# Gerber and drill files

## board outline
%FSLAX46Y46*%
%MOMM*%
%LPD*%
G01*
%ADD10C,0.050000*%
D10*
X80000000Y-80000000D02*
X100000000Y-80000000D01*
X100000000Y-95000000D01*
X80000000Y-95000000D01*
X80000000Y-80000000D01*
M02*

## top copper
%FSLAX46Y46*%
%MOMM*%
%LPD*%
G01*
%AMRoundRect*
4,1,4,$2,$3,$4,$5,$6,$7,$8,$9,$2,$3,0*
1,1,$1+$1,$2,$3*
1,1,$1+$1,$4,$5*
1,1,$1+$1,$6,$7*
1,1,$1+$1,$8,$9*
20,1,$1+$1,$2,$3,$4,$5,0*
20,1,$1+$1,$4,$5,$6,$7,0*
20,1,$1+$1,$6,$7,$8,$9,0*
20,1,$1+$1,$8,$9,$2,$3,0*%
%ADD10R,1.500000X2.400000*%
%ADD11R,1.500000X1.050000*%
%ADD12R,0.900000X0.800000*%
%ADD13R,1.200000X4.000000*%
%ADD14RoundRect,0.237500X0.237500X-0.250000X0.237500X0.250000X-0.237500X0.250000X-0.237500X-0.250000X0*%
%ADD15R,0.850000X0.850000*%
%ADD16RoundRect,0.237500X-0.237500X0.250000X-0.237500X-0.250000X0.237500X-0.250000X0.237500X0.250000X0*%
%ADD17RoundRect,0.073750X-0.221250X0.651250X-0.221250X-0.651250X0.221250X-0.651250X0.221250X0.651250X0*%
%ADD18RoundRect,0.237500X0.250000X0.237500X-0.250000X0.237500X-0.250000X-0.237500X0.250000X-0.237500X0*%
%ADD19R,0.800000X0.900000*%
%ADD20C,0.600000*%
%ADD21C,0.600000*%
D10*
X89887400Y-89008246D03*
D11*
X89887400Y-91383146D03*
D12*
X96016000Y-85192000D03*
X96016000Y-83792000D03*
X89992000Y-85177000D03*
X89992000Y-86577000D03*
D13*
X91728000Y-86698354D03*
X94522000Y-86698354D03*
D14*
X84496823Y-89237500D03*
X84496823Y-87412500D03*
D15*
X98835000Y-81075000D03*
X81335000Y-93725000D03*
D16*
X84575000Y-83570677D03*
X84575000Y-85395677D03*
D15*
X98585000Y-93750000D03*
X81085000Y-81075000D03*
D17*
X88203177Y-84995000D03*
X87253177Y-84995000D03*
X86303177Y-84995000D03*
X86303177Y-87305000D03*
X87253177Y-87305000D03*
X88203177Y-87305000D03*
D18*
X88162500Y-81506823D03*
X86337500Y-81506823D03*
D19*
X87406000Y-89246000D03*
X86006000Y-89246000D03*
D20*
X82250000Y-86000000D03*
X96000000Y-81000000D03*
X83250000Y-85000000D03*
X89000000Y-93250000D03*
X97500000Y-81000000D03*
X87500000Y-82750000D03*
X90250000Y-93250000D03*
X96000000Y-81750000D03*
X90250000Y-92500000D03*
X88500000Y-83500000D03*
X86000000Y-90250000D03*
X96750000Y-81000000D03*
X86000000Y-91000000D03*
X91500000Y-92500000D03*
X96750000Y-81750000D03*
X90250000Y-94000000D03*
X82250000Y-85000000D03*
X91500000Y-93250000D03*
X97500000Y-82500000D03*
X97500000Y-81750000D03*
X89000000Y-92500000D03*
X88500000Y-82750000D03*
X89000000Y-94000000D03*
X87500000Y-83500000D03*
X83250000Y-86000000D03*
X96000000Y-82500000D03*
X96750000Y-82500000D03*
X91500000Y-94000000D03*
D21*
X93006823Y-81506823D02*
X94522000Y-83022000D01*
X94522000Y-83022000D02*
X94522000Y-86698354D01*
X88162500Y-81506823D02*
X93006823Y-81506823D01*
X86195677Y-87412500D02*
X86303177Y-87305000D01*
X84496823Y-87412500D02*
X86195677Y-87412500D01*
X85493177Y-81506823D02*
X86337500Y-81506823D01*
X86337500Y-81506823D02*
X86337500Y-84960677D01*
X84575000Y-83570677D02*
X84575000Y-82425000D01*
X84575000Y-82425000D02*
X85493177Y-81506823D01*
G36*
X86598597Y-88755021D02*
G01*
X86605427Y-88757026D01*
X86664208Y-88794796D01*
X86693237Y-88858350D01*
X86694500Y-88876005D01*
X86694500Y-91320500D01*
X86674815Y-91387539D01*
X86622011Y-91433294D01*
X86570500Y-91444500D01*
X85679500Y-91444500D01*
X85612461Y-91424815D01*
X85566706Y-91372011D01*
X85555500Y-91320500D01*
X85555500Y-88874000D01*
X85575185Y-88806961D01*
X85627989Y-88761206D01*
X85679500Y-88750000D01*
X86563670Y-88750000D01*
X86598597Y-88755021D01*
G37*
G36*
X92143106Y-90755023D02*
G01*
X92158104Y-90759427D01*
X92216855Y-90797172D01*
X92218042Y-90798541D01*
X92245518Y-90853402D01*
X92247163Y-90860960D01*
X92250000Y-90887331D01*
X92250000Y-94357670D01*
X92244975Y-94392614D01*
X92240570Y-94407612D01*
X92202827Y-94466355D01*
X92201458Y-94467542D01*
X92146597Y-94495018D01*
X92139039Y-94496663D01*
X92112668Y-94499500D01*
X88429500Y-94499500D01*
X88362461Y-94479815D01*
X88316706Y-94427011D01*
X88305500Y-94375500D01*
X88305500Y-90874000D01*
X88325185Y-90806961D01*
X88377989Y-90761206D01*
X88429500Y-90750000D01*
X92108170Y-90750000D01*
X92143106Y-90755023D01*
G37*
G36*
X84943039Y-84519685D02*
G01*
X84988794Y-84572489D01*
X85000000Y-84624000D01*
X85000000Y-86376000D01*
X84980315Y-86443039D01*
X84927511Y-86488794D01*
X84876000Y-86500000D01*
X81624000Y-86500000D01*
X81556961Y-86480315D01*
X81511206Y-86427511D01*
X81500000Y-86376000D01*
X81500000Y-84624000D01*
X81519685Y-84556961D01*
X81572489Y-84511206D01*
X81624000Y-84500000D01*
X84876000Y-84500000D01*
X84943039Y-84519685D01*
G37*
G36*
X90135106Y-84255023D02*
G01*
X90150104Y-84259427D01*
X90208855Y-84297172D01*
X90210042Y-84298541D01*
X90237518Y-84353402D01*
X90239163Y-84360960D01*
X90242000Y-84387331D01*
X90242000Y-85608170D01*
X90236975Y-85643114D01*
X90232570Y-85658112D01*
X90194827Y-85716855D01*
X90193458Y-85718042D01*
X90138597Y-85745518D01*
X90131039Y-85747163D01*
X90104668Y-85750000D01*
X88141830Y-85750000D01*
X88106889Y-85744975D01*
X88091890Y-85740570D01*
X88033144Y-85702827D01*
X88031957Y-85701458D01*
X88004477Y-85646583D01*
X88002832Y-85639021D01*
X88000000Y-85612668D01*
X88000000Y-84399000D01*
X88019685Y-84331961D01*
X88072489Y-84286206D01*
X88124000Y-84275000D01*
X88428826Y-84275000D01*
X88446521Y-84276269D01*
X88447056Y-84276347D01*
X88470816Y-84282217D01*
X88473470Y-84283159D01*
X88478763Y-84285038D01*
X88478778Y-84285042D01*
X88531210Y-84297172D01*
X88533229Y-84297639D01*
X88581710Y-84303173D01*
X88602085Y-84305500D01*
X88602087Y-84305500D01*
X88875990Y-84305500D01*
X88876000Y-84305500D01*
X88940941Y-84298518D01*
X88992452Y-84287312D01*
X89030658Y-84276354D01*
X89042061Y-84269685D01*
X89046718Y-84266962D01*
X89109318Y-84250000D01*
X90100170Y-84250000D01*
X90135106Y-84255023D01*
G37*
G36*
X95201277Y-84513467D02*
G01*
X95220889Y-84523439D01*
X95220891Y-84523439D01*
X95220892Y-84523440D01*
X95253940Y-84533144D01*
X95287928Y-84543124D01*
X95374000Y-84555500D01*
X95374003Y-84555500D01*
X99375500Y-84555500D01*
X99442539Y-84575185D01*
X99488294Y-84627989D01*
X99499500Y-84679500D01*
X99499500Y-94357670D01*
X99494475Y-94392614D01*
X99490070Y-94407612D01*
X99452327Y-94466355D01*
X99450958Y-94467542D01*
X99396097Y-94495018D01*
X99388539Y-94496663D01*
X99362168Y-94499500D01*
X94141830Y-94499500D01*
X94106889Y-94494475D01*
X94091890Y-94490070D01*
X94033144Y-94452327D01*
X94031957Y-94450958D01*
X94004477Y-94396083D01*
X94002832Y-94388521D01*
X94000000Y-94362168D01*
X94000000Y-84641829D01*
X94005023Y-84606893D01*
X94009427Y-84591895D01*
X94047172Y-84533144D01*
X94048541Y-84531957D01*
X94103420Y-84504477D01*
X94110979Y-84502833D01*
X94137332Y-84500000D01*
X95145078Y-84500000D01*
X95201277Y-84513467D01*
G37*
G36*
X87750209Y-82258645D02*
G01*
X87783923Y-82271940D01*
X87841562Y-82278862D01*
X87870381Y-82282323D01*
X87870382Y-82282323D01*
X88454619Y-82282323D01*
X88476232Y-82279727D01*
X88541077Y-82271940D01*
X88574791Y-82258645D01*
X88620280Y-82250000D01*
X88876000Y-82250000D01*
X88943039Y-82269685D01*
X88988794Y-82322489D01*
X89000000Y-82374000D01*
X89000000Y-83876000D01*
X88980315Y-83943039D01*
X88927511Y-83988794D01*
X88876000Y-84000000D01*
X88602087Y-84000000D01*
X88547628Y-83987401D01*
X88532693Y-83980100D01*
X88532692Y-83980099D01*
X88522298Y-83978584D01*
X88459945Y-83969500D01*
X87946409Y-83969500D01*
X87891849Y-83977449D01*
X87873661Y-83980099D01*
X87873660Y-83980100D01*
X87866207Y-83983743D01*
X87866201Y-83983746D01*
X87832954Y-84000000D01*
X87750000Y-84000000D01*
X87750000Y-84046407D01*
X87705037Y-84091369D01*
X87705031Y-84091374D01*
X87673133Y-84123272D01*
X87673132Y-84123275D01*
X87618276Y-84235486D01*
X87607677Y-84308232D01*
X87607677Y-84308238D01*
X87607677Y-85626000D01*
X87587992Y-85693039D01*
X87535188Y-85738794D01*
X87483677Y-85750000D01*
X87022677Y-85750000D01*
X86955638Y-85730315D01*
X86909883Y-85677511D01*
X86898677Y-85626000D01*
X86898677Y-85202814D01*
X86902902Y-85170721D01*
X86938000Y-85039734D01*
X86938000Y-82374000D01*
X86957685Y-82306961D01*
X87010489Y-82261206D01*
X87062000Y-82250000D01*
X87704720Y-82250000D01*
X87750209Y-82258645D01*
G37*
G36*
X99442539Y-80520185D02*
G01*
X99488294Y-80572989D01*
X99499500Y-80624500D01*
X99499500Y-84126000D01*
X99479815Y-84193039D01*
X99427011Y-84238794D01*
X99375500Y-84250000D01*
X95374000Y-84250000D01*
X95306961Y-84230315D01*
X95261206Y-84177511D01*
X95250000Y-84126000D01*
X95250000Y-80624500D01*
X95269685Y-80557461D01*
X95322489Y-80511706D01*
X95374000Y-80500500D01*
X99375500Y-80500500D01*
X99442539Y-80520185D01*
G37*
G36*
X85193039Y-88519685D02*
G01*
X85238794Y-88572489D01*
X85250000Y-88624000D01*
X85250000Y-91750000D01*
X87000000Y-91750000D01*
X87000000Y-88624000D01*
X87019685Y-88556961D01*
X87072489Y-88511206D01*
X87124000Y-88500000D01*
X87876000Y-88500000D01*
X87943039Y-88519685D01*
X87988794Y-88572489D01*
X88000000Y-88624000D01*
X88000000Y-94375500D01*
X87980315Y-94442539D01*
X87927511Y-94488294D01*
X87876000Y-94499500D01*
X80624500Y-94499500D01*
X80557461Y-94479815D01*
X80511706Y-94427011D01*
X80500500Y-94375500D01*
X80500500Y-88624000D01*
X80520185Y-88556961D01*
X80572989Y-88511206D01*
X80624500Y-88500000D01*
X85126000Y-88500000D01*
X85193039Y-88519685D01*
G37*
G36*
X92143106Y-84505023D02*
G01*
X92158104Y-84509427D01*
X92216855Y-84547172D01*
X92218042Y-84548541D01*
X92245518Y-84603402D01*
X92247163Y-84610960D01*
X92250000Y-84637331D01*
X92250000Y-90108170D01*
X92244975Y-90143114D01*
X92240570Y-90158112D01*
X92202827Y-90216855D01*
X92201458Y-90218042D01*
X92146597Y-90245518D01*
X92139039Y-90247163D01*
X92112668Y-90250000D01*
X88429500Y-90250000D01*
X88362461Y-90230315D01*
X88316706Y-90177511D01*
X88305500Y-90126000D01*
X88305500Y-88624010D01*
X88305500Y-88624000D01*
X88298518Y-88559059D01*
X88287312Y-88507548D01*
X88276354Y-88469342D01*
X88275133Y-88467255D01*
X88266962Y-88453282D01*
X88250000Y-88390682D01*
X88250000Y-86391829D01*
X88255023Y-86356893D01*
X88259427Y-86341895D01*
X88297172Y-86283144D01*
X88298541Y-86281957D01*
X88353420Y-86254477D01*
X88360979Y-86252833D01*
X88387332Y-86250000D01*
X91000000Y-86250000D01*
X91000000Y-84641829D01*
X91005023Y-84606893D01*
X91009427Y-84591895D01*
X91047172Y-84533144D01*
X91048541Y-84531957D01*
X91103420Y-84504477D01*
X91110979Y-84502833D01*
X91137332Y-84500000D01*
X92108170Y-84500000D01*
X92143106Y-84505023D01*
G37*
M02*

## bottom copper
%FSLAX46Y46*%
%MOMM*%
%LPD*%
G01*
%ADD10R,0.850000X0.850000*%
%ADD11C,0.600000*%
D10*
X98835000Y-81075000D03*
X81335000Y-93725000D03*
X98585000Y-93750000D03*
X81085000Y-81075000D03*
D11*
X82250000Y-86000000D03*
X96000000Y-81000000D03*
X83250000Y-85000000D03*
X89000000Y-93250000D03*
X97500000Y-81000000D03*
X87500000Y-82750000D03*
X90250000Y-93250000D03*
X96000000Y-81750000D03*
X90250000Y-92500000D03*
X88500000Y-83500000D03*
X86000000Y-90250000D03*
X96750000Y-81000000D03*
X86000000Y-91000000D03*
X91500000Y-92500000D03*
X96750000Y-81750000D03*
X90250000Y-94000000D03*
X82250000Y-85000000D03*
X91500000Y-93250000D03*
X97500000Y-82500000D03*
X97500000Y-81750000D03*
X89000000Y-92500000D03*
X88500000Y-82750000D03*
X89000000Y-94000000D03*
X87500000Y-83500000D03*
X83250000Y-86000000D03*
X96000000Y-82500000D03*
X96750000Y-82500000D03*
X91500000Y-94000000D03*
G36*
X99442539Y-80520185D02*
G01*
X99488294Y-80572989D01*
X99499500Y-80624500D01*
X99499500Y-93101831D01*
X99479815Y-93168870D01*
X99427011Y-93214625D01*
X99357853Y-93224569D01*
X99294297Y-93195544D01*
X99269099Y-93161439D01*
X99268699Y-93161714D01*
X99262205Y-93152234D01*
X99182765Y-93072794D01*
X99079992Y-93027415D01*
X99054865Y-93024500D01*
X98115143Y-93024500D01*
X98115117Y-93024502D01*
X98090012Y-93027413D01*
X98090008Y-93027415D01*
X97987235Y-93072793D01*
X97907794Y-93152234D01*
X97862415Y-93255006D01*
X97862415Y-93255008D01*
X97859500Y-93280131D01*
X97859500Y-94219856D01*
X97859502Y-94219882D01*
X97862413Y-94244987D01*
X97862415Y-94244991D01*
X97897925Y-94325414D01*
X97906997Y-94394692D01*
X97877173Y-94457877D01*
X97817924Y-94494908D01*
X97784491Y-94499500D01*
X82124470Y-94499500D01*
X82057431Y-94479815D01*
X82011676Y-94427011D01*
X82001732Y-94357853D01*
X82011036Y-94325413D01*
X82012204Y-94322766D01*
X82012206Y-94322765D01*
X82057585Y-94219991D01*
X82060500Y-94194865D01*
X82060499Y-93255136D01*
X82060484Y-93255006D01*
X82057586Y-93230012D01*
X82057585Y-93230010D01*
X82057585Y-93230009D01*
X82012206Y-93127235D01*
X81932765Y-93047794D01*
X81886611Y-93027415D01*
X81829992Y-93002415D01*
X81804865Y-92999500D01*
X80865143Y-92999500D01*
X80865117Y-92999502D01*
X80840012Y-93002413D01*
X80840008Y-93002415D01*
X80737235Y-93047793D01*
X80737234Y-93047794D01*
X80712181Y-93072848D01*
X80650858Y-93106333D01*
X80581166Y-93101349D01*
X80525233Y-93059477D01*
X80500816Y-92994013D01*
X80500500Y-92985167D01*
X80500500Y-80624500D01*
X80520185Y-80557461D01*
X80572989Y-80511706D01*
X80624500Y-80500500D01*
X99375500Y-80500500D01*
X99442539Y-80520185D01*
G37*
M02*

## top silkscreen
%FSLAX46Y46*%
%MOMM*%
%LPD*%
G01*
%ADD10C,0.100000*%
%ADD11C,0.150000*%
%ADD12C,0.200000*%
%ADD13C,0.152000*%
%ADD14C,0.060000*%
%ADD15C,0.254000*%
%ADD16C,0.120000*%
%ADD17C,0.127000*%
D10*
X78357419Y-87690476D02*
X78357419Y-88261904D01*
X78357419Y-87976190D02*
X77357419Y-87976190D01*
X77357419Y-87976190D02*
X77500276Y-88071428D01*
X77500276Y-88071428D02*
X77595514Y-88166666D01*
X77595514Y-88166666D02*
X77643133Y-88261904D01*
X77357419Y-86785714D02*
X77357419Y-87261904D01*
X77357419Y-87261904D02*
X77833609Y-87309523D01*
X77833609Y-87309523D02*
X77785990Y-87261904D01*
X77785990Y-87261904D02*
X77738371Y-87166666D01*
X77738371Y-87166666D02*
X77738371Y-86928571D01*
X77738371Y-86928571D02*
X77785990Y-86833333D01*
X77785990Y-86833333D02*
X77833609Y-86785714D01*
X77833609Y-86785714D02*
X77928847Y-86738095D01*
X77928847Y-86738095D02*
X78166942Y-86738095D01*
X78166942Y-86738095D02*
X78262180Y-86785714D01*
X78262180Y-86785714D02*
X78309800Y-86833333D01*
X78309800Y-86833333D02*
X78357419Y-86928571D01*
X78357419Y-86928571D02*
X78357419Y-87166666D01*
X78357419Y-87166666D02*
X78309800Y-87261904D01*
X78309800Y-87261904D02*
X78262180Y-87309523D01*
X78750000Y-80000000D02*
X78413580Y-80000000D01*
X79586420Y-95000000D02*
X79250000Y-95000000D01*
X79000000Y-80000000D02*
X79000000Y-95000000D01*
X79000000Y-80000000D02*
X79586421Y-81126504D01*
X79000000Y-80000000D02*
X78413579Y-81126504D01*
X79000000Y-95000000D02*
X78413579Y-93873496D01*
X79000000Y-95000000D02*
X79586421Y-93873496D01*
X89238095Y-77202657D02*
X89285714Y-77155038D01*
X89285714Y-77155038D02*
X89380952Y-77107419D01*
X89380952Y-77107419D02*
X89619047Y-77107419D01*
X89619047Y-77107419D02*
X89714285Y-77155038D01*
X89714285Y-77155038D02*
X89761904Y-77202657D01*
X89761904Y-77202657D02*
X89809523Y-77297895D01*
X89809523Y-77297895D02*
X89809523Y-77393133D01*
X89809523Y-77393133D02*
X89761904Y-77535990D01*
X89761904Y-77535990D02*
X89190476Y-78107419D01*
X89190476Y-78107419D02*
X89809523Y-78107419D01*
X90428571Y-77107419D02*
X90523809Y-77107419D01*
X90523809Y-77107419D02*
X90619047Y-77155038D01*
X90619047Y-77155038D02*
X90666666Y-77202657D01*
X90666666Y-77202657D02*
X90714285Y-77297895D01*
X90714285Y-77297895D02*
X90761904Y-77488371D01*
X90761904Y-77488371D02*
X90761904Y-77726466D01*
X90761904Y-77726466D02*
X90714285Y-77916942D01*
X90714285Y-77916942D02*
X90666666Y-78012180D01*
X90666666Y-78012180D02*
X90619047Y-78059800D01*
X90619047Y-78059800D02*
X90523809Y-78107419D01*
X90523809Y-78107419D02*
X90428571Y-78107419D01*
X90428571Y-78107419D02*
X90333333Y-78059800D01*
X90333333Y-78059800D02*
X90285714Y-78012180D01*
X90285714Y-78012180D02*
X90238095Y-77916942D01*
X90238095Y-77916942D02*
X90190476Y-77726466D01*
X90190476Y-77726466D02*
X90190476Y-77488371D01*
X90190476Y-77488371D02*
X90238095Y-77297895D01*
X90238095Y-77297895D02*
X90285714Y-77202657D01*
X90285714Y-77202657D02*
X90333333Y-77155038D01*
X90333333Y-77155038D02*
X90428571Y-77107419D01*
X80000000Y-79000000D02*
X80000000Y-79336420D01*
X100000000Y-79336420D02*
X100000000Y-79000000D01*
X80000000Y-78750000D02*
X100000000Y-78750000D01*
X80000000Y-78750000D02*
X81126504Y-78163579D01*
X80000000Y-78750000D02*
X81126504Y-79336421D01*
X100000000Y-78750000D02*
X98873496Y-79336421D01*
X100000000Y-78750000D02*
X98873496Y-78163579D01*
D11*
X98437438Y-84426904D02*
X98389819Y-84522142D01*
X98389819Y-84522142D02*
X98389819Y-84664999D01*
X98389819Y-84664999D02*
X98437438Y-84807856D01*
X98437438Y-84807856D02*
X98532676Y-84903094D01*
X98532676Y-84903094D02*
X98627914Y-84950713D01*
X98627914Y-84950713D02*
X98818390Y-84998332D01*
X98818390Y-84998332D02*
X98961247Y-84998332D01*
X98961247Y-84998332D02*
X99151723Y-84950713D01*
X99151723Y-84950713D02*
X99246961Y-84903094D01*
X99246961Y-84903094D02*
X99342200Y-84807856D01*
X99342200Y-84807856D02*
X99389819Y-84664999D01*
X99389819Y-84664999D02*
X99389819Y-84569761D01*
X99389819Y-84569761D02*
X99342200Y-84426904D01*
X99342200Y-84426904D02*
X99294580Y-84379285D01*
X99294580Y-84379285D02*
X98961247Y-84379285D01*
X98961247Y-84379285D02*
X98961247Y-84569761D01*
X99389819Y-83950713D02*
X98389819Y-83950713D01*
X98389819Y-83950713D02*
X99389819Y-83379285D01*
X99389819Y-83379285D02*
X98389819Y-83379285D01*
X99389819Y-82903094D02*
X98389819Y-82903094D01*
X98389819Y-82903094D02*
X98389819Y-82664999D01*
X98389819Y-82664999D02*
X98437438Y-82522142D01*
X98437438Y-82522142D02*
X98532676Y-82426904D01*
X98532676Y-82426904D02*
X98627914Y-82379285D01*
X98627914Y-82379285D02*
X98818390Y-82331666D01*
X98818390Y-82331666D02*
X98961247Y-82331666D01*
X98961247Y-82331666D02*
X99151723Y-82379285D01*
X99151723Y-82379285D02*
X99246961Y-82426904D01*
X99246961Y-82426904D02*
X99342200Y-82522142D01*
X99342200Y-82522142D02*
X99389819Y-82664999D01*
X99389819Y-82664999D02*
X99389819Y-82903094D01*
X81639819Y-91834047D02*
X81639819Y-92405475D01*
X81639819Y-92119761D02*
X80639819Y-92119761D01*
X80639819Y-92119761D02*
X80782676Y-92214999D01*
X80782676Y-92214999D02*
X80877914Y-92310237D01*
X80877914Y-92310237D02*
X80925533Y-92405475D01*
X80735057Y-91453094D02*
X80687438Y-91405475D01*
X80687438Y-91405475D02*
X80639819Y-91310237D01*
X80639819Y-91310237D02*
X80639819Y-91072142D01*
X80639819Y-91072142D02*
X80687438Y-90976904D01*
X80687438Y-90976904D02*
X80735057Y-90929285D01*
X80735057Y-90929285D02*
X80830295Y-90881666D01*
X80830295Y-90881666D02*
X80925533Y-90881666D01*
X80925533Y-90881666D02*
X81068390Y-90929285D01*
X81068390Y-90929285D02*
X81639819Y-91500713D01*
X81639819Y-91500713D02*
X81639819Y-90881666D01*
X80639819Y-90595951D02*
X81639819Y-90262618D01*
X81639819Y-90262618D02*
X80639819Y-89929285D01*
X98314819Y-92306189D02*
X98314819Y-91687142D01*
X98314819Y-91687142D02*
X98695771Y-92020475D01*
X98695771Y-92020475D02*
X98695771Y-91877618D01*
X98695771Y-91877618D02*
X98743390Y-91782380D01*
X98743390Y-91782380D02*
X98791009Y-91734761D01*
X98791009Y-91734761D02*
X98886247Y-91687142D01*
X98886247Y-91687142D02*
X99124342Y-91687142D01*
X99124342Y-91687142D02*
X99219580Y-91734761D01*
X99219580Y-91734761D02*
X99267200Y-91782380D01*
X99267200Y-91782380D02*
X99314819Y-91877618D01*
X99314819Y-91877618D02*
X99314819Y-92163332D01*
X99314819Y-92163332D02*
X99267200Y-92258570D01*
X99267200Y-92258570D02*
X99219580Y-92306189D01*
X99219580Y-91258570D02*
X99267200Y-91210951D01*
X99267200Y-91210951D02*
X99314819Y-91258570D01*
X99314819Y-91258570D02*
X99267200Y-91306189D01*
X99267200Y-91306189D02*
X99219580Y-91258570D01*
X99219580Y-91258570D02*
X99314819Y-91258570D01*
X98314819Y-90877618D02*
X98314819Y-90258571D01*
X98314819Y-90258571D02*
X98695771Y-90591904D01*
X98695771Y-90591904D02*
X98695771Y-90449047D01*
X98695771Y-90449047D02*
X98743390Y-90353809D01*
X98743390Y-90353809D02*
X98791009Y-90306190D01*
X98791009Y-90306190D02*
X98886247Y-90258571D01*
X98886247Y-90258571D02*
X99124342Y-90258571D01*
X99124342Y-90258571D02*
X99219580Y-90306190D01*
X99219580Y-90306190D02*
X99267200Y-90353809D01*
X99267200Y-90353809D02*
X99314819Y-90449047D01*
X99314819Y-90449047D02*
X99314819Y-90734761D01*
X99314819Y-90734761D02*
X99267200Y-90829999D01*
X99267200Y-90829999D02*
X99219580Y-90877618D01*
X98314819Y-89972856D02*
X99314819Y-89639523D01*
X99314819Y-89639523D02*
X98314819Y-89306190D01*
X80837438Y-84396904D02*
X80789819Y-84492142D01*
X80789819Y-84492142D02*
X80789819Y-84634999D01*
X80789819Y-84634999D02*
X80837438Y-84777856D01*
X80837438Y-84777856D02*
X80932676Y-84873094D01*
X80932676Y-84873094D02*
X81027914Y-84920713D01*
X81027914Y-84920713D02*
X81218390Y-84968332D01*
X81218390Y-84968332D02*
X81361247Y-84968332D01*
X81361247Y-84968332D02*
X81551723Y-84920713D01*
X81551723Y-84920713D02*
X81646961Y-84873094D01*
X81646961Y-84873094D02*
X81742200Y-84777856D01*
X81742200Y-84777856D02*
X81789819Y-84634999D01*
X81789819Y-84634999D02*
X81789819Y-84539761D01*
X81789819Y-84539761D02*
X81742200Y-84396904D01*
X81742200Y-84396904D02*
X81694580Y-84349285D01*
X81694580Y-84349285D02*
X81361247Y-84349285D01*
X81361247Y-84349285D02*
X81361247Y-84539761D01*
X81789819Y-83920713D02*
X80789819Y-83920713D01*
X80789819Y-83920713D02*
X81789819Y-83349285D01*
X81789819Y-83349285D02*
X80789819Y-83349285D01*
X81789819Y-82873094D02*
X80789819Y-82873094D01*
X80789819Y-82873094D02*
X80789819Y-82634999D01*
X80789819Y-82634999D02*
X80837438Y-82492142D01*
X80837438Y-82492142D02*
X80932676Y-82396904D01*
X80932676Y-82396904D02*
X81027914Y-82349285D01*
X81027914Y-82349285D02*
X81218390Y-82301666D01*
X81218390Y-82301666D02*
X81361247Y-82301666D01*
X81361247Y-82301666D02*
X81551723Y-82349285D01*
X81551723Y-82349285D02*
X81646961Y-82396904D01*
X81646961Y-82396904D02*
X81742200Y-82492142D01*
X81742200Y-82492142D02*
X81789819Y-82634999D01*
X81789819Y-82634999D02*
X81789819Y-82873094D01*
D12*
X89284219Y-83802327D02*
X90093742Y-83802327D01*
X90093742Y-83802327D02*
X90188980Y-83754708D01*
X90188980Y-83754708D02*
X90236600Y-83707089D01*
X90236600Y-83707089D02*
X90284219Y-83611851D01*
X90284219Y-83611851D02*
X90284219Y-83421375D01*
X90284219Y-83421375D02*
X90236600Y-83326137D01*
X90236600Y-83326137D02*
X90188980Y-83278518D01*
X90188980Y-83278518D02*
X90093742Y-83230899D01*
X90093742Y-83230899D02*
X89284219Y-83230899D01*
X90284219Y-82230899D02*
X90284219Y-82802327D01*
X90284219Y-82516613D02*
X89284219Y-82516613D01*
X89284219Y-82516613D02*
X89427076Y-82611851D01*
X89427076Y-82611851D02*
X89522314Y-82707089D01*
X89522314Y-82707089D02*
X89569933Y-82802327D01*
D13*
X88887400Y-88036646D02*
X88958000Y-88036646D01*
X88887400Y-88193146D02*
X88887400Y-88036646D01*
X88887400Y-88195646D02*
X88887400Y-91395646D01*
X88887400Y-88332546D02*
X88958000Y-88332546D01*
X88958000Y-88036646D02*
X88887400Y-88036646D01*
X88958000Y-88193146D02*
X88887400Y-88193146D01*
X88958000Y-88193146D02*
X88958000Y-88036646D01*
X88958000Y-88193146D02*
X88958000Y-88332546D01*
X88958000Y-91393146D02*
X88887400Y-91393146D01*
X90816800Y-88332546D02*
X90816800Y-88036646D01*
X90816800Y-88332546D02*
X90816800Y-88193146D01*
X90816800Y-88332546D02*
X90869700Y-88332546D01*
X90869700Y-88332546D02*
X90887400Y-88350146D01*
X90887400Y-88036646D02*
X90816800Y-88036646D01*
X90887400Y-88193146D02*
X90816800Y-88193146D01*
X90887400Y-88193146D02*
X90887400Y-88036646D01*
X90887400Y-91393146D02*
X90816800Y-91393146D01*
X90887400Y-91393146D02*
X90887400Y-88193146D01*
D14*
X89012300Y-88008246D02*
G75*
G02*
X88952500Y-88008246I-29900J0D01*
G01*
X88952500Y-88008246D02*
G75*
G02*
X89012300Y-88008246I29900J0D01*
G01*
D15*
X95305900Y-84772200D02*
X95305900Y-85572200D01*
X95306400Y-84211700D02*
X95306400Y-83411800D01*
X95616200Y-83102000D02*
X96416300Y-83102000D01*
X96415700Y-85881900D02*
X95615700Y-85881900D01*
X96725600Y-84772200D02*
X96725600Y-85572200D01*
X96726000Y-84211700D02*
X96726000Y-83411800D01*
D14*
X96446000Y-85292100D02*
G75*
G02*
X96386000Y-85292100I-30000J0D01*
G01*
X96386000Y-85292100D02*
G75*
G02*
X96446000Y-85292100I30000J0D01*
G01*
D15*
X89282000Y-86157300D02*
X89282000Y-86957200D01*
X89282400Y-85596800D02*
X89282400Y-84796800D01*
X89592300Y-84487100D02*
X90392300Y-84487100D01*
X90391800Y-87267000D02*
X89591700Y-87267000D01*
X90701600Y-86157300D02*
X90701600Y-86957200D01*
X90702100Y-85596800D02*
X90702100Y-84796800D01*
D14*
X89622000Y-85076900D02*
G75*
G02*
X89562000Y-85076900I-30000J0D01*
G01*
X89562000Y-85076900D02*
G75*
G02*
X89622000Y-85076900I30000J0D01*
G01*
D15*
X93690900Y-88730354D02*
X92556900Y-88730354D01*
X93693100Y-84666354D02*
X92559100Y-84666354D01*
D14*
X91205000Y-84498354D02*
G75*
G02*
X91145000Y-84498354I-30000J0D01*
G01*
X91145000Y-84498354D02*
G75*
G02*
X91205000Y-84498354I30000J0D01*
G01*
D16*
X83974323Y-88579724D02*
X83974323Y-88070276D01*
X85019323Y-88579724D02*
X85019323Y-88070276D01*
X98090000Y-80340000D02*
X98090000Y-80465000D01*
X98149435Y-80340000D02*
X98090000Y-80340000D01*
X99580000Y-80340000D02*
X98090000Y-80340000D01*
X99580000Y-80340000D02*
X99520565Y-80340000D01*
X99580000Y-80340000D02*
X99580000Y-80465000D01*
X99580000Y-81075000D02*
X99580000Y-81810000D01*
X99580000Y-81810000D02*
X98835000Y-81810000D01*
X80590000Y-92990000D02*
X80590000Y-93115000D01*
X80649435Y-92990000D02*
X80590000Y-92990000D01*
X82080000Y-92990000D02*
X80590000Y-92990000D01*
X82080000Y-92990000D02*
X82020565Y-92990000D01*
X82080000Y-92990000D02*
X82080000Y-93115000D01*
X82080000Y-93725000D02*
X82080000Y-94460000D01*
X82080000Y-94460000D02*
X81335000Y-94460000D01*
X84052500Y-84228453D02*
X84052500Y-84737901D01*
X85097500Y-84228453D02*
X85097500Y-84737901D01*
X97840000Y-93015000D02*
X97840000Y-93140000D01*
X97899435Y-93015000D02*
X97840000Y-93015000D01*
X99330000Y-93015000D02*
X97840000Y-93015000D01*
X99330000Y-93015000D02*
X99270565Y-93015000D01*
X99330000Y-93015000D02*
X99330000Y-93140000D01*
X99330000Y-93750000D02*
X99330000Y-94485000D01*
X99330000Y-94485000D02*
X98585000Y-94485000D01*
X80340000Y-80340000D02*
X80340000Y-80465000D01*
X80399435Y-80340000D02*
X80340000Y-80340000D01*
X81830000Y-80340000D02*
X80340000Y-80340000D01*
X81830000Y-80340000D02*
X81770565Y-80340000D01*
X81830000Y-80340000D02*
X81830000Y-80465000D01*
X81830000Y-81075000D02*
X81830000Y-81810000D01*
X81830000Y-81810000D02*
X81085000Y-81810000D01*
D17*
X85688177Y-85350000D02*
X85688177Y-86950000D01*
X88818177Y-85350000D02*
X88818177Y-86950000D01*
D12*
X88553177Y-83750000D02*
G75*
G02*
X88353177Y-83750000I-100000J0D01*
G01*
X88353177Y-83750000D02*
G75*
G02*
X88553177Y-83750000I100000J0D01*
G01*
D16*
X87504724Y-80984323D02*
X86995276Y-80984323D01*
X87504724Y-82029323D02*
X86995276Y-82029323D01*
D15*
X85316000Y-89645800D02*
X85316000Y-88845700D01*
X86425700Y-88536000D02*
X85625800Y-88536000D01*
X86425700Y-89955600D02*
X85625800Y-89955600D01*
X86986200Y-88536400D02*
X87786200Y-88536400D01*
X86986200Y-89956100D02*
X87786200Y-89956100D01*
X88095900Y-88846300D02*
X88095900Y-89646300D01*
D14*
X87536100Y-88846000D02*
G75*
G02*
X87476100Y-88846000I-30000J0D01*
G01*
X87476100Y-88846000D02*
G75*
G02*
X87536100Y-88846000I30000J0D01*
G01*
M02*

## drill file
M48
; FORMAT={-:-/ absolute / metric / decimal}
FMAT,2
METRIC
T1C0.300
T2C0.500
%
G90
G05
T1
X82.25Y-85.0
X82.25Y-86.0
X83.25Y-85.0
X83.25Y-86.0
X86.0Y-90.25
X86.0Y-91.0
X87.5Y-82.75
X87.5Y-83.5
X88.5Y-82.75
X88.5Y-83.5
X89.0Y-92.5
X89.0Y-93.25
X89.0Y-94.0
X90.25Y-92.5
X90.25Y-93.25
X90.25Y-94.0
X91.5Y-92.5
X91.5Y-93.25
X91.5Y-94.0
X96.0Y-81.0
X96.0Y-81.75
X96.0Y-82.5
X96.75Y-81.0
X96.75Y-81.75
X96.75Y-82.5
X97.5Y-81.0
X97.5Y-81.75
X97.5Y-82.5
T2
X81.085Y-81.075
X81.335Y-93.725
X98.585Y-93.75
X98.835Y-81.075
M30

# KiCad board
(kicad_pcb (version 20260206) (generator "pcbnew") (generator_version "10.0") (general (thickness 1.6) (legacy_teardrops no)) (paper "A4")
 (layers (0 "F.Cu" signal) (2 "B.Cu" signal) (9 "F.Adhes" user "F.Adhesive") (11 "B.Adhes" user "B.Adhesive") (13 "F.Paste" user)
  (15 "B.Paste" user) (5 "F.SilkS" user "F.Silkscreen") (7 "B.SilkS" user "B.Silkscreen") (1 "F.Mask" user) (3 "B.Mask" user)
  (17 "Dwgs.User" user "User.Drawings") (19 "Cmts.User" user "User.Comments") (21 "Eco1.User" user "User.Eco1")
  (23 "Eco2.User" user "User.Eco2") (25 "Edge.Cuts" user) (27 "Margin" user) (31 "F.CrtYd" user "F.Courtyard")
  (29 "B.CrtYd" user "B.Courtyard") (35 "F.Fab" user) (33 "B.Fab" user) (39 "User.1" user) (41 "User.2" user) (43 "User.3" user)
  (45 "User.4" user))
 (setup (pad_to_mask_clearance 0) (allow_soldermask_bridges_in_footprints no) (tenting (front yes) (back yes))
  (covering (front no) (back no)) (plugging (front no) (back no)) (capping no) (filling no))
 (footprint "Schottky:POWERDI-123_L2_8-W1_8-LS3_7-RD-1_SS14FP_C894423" (layer "F.Cu") (at 89.8874 90.195646 -90)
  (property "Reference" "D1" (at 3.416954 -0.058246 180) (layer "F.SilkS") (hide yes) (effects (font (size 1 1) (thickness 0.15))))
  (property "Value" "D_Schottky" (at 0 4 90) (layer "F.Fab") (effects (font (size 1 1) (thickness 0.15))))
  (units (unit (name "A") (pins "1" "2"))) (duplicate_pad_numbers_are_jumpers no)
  (fp_line (start -2.159 1) (end -2.159 0.9294) (stroke (width 0.152) (type solid)) (layer "F.SilkS"))
  (fp_line (start -2.0025 1) (end -2.159 1) (stroke (width 0.152) (type solid)) (layer "F.SilkS"))
  (fp_line (start -2 1) (end 1.2 1) (stroke (width 0.152) (type solid)) (layer "F.SilkS"))
  (fp_line (start -1.8631 1) (end -1.8631 0.9294) (stroke (width 0.152) (type solid)) (layer "F.SilkS"))
  (fp_line (start -2.159 0.9294) (end -2.159 1) (stroke (width 0.152) (type solid)) (layer "F.SilkS"))
  (fp_line (start -2.0025 0.9294) (end -2.0025 1) (stroke (width 0.152) (type solid)) (layer "F.SilkS"))
  (fp_line (start -2.0025 0.9294) (end -2.159 0.9294) (stroke (width 0.152) (type solid)) (layer "F.SilkS"))
  (fp_line (start -2.0025 0.9294) (end -1.8631 0.9294) (stroke (width 0.152) (type solid)) (layer "F.SilkS"))
  (fp_line (start 1.1975 0.9294) (end 1.1975 1) (stroke (width 0.152) (type solid)) (layer "F.SilkS"))
  (fp_line (start -1.8631 -0.9294) (end -2.159 -0.9294) (stroke (width 0.152) (type solid)) (layer "F.SilkS"))
  (fp_line (start -1.8631 -0.9294) (end -2.0025 -0.9294) (stroke (width 0.152) (type solid)) (layer "F.SilkS"))
  (fp_line (start -1.8631 -0.9294) (end -1.8631 -0.9823) (stroke (width 0.152) (type solid)) (layer "F.SilkS"))
  (fp_line (start -1.8631 -0.9823) (end -1.8455 -1) (stroke (width 0.152) (type solid)) (layer "F.SilkS"))
  (fp_line (start -2.159 -1) (end -2.159 -0.9294) (stroke (width 0.152) (type solid)) (layer "F.SilkS"))
  (fp_line (start -2.0025 -1) (end -2.0025 -0.9294) (stroke (width 0.152) (type solid)) (layer "F.SilkS"))
  (fp_line (start -2.0025 -1) (end -2.159 -1) (stroke (width 0.152) (type solid)) (layer "F.SilkS"))
  (fp_line (start 1.1975 -1) (end 1.1975 -0.9294) (stroke (width 0.152) (type solid)) (layer "F.SilkS"))
  (fp_line (start 1.1975 -1) (end -2.0025 -1) (stroke (width 0.152) (type solid)) (layer "F.SilkS"))
  (fp_circle (center -2.1874 0.905) (end -2.1575 0.905) (stroke (width 0.06) (type solid)) (fill no) (layer "F.SilkS"))
  (pad "1" smd rect (at -1.1874 0 90) (size 2.4 1.5) (layers "F.Cu" "F.Mask" "F.Paste") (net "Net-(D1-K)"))
  (pad "2" smd rect (at 1.1875 0 90) (size 1.05 1.5) (layers "F.Cu" "F.Mask" "F.Paste") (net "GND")))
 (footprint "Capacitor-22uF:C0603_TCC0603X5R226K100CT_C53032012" (layer "F.Cu") (at 96.016 84.492 90)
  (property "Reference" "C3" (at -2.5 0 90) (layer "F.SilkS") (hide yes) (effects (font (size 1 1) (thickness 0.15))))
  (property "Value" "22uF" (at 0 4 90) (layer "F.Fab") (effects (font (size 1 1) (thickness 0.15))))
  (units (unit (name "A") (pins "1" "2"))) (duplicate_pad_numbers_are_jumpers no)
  (fp_line (start -0.2802 -0.7101) (end -1.0802 -0.7101) (stroke (width 0.254) (type solid)) (layer "F.SilkS"))
  (fp_line (start 0.2803 -0.7096) (end 1.0802 -0.7096) (stroke (width 0.254) (type solid)) (layer "F.SilkS"))
  (fp_line (start 1.39 -0.3998) (end 1.39 0.4003) (stroke (width 0.254) (type solid)) (layer "F.SilkS"))
  (fp_line (start -1.3899 0.3997) (end -1.3899 -0.4003) (stroke (width 0.254) (type solid)) (layer "F.SilkS"))
  (fp_line (start -0.2802 0.7096) (end -1.0802 0.7096) (stroke (width 0.254) (type solid)) (layer "F.SilkS"))
  (fp_line (start 0.2803 0.71) (end 1.0802 0.71) (stroke (width 0.254) (type solid)) (layer "F.SilkS"))
  (fp_circle (center -0.8001 0.4) (end -0.7701 0.4) (stroke (width 0.06) (type solid)) (fill no) (layer "F.SilkS"))
  (pad "1" smd rect (at -0.7 0 90) (size 0.8 0.9) (layers "F.Cu" "F.Mask" "F.Paste") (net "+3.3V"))
  (pad "2" smd rect (at 0.7 0 90) (size 0.8 0.9) (layers "F.Cu" "F.Mask" "F.Paste") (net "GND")))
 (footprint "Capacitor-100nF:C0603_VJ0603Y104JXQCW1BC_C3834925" (layer "F.Cu") (at 89.992 85.877 -90)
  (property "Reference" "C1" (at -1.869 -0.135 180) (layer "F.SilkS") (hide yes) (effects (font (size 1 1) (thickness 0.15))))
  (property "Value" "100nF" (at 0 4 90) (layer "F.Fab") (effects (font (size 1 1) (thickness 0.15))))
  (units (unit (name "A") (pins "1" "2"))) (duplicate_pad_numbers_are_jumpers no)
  (fp_line (start 0.2803 0.71) (end 1.0802 0.71) (stroke (width 0.254) (type solid)) (layer "F.SilkS"))
  (fp_line (start -0.2802 0.7096) (end -1.0802 0.7096) (stroke (width 0.254) (type solid)) (layer "F.SilkS"))
  (fp_line (start -1.3899 0.3997) (end -1.3899 -0.4003) (stroke (width 0.254) (type solid)) (layer "F.SilkS"))
  (fp_line (start 1.39 -0.3998) (end 1.39 0.4003) (stroke (width 0.254) (type solid)) (layer "F.SilkS"))
  (fp_line (start 0.2803 -0.7096) (end 1.0802 -0.7096) (stroke (width 0.254) (type solid)) (layer "F.SilkS"))
  (fp_line (start -0.2802 -0.7101) (end -1.0802 -0.7101) (stroke (width 0.254) (type solid)) (layer "F.SilkS"))
  (fp_circle (center -0.8001 0.4) (end -0.7701 0.4) (stroke (width 0.06) (type solid)) (fill no) (layer "F.SilkS"))
  (pad "1" smd rect (at -0.7 0 270) (size 0.8 0.9) (layers "F.Cu" "F.Mask" "F.Paste") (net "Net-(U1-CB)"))
  (pad "2" smd rect (at 0.7 0 270) (size 0.8 0.9) (layers "F.Cu" "F.Mask" "F.Paste") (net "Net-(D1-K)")))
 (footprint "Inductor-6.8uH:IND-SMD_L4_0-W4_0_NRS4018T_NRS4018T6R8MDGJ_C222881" (layer "F.Cu") (at 93.125 86.698354 180)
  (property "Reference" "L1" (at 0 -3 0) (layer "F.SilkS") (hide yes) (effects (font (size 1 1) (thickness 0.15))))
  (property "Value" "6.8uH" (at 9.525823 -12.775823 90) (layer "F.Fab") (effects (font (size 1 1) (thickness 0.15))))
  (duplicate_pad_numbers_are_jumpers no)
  (fp_line (start -0.5659 -2.032) (end 0.5681 -2.032) (stroke (width 0.254) (type solid)) (layer "F.SilkS"))
  (fp_line (start -0.5681 2.032) (end 0.5659 2.032) (stroke (width 0.254) (type solid)) (layer "F.SilkS"))
  (fp_circle (center 1.95 2.2) (end 1.98 2.2) (stroke (width 0.06) (type solid)) (fill no) (layer "F.SilkS"))
  (pad "1" smd rect (at 1.397 0 180) (size 1.2 4) (layers "F.Cu" "F.Mask" "F.Paste") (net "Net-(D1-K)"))
  (pad "2" smd rect (at -1.397 0 180) (size 1.2 4) (layers "F.Cu" "F.Mask" "F.Paste") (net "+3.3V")))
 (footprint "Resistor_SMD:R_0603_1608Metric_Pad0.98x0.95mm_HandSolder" (layer "F.Cu") (at 84.496823 88.325 90)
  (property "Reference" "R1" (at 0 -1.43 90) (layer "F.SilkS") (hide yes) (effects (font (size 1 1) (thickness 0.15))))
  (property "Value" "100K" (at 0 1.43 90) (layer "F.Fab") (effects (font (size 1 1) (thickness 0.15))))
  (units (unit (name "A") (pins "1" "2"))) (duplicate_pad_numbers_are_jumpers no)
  (fp_line (start -0.254724 -0.5225) (end 0.254724 -0.5225) (stroke (width 0.12) (type solid)) (layer "F.SilkS"))
  (fp_line (start -0.254724 0.5225) (end 0.254724 0.5225) (stroke (width 0.12) (type solid)) (layer "F.SilkS"))
  (pad "1" smd roundrect (at -0.9125 0 90) (size 0.975 0.95) (layers "F.Cu" "F.Mask" "F.Paste") (roundrect_rratio 0.25) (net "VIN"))
  (pad "2" smd roundrect (at 0.9125 0 90) (size 0.975 0.95) (layers "F.Cu" "F.Mask" "F.Paste") (roundrect_rratio 0.25) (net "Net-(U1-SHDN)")))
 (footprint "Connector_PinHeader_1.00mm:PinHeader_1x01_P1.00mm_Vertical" (layer "F.Cu") (at 98.835 81.075 180)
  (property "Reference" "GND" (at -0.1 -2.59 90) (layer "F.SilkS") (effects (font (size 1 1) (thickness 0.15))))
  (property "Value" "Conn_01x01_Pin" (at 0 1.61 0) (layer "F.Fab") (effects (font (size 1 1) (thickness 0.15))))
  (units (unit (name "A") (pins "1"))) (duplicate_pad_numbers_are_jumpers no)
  (fp_line (start 0.745 0.735) (end 0.745 0.61) (stroke (width 0.12) (type solid)) (layer "F.SilkS"))
  (fp_line (start 0.685565 0.735) (end 0.745 0.735) (stroke (width 0.12) (type solid)) (layer "F.SilkS"))
  (fp_line (start -0.745 0.735) (end 0.745 0.735) (stroke (width 0.12) (type solid)) (layer "F.SilkS"))
  (fp_line (start -0.745 0.735) (end -0.685565 0.735) (stroke (width 0.12) (type solid)) (layer "F.SilkS"))
  (fp_line (start -0.745 0.735) (end -0.745 0.61) (stroke (width 0.12) (type solid)) (layer "F.SilkS"))
  (fp_line (start -0.745 0) (end -0.745 -0.735) (stroke (width 0.12) (type solid)) (layer "F.SilkS"))
  (fp_line (start -0.745 -0.735) (end 0 -0.735) (stroke (width 0.12) (type solid)) (layer "F.SilkS"))
  (pad "1" thru_hole rect (at 0 0 180) (size 0.85 0.85) (drill 0.5) (layers "*.Cu" "*.Mask") (remove_unused_layers no) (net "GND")))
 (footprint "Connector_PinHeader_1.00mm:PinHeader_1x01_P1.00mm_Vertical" (layer "F.Cu") (at 81.335 93.725 180)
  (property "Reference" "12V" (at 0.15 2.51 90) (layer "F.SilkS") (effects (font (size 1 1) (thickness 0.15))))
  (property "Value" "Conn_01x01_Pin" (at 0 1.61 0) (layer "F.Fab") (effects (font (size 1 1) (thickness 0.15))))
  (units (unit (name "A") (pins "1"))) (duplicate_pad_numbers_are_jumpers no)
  (fp_line (start 0.745 0.735) (end 0.745 0.61) (stroke (width 0.12) (type solid)) (layer "F.SilkS"))
  (fp_line (start 0.685565 0.735) (end 0.745 0.735) (stroke (width 0.12) (type solid)) (layer "F.SilkS"))
  (fp_line (start -0.745 0.735) (end 0.745 0.735) (stroke (width 0.12) (type solid)) (layer "F.SilkS"))
  (fp_line (start -0.745 0.735) (end -0.685565 0.735) (stroke (width 0.12) (type solid)) (layer "F.SilkS"))
  (fp_line (start -0.745 0.735) (end -0.745 0.61) (stroke (width 0.12) (type solid)) (layer "F.SilkS"))
  (fp_line (start -0.745 0) (end -0.745 -0.735) (stroke (width 0.12) (type solid)) (layer "F.SilkS"))
  (fp_line (start -0.745 -0.735) (end 0 -0.735) (stroke (width 0.12) (type solid)) (layer "F.SilkS"))
  (pad "1" thru_hole rect (at 0 0 180) (size 0.85 0.85) (drill 0.5) (layers "*.Cu" "*.Mask") (remove_unused_layers no) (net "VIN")))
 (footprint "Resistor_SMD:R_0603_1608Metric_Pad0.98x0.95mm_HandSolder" (layer "F.Cu") (at 84.575 84.483177 -90)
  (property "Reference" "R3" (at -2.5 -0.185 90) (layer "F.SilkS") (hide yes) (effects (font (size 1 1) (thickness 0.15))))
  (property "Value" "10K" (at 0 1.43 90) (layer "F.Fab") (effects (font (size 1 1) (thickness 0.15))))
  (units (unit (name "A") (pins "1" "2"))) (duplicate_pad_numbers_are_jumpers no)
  (fp_line (start -0.254724 0.5225) (end 0.254724 0.5225) (stroke (width 0.12) (type solid)) (layer "F.SilkS"))
  (fp_line (start -0.254724 -0.5225) (end 0.254724 -0.5225) (stroke (width 0.12) (type solid)) (layer "F.SilkS"))
  (pad "1" smd roundrect (at -0.9125 0 270) (size 0.975 0.95) (layers "F.Cu" "F.Mask" "F.Paste") (roundrect_rratio 0.25) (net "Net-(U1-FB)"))
  (pad "2" smd roundrect (at 0.9125 0 270) (size 0.975 0.95) (layers "F.Cu" "F.Mask" "F.Paste") (roundrect_rratio 0.25) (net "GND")))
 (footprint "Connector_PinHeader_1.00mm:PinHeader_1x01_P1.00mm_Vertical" (layer "F.Cu") (at 98.585 93.75 180)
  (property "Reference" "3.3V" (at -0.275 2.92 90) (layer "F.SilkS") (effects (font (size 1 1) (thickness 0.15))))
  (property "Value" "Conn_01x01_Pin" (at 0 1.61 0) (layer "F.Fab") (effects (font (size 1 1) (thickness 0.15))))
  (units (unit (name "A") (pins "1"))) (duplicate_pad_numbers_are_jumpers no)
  (fp_line (start 0.745 0.735) (end 0.745 0.61) (stroke (width 0.12) (type solid)) (layer "F.SilkS"))
  (fp_line (start 0.685565 0.735) (end 0.745 0.735) (stroke (width 0.12) (type solid)) (layer "F.SilkS"))
  (fp_line (start -0.745 0.735) (end 0.745 0.735) (stroke (width 0.12) (type solid)) (layer "F.SilkS"))
  (fp_line (start -0.745 0.735) (end -0.685565 0.735) (stroke (width 0.12) (type solid)) (layer "F.SilkS"))
  (fp_line (start -0.745 0.735) (end -0.745 0.61) (stroke (width 0.12) (type solid)) (layer "F.SilkS"))
  (fp_line (start -0.745 0) (end -0.745 -0.735) (stroke (width 0.12) (type solid)) (layer "F.SilkS"))
  (fp_line (start -0.745 -0.735) (end 0 -0.735) (stroke (width 0.12) (type solid)) (layer "F.SilkS"))
  (pad "1" thru_hole rect (at 0 0 180) (size 0.85 0.85) (drill 0.5) (layers "*.Cu" "*.Mask") (remove_unused_layers no) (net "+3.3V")))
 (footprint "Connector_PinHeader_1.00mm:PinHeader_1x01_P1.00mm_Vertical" (layer "F.Cu") (at 81.085 81.075 180)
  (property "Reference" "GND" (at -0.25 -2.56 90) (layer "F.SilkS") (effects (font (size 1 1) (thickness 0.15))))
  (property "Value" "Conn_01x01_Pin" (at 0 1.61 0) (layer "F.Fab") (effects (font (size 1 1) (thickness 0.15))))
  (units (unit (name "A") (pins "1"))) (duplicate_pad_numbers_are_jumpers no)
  (fp_line (start 0.745 0.735) (end 0.745 0.61) (stroke (width 0.12) (type solid)) (layer "F.SilkS"))
  (fp_line (start 0.685565 0.735) (end 0.745 0.735) (stroke (width 0.12) (type solid)) (layer "F.SilkS"))
  (fp_line (start -0.745 0.735) (end 0.745 0.735) (stroke (width 0.12) (type solid)) (layer "F.SilkS"))
  (fp_line (start -0.745 0.735) (end -0.685565 0.735) (stroke (width 0.12) (type solid)) (layer "F.SilkS"))
  (fp_line (start -0.745 0.735) (end -0.745 0.61) (stroke (width 0.12) (type solid)) (layer "F.SilkS"))
  (fp_line (start -0.745 0) (end -0.745 -0.735) (stroke (width 0.12) (type solid)) (layer "F.SilkS"))
  (fp_line (start -0.745 -0.735) (end 0 -0.735) (stroke (width 0.12) (type solid)) (layer "F.SilkS"))
  (pad "1" thru_hole rect (at 0 0 180) (size 0.85 0.85) (drill 0.5) (layers "*.Cu" "*.Mask") (remove_unused_layers no) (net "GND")))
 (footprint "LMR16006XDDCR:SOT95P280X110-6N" (layer "F.Cu") (at 87.253177 86.15 -90)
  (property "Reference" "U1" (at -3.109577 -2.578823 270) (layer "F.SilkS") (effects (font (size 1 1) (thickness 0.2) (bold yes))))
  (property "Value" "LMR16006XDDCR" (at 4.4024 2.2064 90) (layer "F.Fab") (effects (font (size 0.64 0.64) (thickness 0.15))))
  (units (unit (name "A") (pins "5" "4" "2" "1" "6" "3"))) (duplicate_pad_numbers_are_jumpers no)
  (fp_line (start -0.8 1.565) (end 0.8 1.565) (stroke (width 0.127) (type solid)) (layer "F.SilkS"))
  (fp_line (start -0.8 -1.565) (end 0.8 -1.565) (stroke (width 0.127) (type solid)) (layer "F.SilkS"))
  (fp_circle (center -2.4 -1.2) (end -2.3 -1.2) (stroke (width 0.2) (type solid)) (fill no) (layer "F.SilkS"))
  (pad "1" smd roundrect (at -1.155 -0.95 270) (size 1.45 0.59) (layers "F.Cu" "F.Mask" "F.Paste") (roundrect_rratio 0.125)
   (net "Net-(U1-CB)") (solder_mask_margin 0.102))
  (pad "2" smd roundrect (at -1.155 0 270) (size 1.45 0.59) (layers "F.Cu" "F.Mask" "F.Paste") (roundrect_rratio 0.125) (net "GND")
   (solder_mask_margin 0.102))
  (pad "3" smd roundrect (at -1.155 0.95 270) (size 1.45 0.59) (layers "F.Cu" "F.Mask" "F.Paste") (roundrect_rratio 0.125)
   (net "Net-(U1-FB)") (solder_mask_margin 0.102))
  (pad "4" smd roundrect (at 1.155 0.95 270) (size 1.45 0.59) (layers "F.Cu" "F.Mask" "F.Paste") (roundrect_rratio 0.125)
   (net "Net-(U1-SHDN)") (solder_mask_margin 0.102))
  (pad "5" smd roundrect (at 1.155 0 270) (size 1.45 0.59) (layers "F.Cu" "F.Mask" "F.Paste") (roundrect_rratio 0.125) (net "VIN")
   (solder_mask_margin 0.102))
  (pad "6" smd roundrect (at 1.155 -0.95 270) (size 1.45 0.59) (layers "F.Cu" "F.Mask" "F.Paste") (roundrect_rratio 0.125)
   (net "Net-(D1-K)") (solder_mask_margin 0.102)))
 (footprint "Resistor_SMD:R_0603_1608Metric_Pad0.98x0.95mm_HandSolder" (layer "F.Cu") (at 87.25 81.506823 180)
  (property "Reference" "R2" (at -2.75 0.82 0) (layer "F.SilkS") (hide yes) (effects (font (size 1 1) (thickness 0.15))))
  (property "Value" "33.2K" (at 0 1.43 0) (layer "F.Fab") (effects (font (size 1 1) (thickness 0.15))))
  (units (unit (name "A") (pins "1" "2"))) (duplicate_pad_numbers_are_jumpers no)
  (fp_line (start -0.254724 0.5225) (end 0.254724 0.5225) (stroke (width 0.12) (type solid)) (layer "F.SilkS"))
  (fp_line (start -0.254724 -0.5225) (end 0.254724 -0.5225) (stroke (width 0.12) (type solid)) (layer "F.SilkS"))
  (pad "1" smd roundrect (at -0.9125 0 180) (size 0.975 0.95) (layers "F.Cu" "F.Mask" "F.Paste") (roundrect_rratio 0.25) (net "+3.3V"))
  (pad "2" smd roundrect (at 0.9125 0 180) (size 0.975 0.95) (layers "F.Cu" "F.Mask" "F.Paste") (roundrect_rratio 0.25) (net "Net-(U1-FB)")))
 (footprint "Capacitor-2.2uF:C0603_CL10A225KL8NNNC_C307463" (layer "F.Cu") (at 86.706 89.246 180)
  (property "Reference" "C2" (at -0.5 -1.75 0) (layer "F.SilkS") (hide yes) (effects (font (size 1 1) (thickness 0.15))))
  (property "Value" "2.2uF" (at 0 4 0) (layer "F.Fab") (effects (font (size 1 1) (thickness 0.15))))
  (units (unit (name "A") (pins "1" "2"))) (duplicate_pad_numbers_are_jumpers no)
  (fp_line (start 1.39 -0.3998) (end 1.39 0.4003) (stroke (width 0.254) (type solid)) (layer "F.SilkS"))
  (fp_line (start 0.2803 0.71) (end 1.0802 0.71) (stroke (width 0.254) (type solid)) (layer "F.SilkS"))
  (fp_line (start 0.2803 -0.7096) (end 1.0802 -0.7096) (stroke (width 0.254) (type solid)) (layer "F.SilkS"))
  (fp_line (start -0.2802 0.7096) (end -1.0802 0.7096) (stroke (width 0.254) (type solid)) (layer "F.SilkS"))
  (fp_line (start -0.2802 -0.7101) (end -1.0802 -0.7101) (stroke (width 0.254) (type solid)) (layer "F.SilkS"))
  (fp_line (start -1.3899 0.3997) (end -1.3899 -0.4003) (stroke (width 0.254) (type solid)) (layer "F.SilkS"))
  (fp_circle (center -0.8001 0.4) (end -0.7701 0.4) (stroke (width 0.06) (type solid)) (fill no) (layer "F.SilkS"))
  (pad "1" smd rect (at -0.7 0 180) (size 0.8 0.9) (layers "F.Cu" "F.Mask" "F.Paste") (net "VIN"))
  (pad "2" smd rect (at 0.7 0 180) (size 0.8 0.9) (layers "F.Cu" "F.Mask" "F.Paste") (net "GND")))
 (gr_rect (start 80 80) (end 100 95) (stroke (width 0.05) (type default)) (fill no) (layer "Edge.Cuts"))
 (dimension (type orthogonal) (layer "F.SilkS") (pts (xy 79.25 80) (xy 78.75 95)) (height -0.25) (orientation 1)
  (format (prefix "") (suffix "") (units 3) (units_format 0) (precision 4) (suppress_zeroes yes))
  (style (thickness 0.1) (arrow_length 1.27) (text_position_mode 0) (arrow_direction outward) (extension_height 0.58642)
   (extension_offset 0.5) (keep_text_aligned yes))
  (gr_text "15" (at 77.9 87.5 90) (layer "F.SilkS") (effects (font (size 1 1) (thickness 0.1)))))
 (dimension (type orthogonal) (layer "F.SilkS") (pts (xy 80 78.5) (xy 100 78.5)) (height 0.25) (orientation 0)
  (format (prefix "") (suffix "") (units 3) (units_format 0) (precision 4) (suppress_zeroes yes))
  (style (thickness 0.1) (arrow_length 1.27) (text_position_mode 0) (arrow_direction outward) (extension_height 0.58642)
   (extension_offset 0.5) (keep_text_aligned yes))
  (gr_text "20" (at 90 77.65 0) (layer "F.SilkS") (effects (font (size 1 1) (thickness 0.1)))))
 (via (at 82.25 86) (size 0.6) (drill 0.3) (layers "F.Cu" "B.Cu") (free yes) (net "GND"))
 (via (at 96 81) (size 0.6) (drill 0.3) (layers "F.Cu" "B.Cu") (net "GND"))
 (via (at 83.25 85) (size 0.6) (drill 0.3) (layers "F.Cu" "B.Cu") (free yes) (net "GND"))
 (via (at 89 93.25) (size 0.6) (drill 0.3) (layers "F.Cu" "B.Cu") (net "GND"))
 (via (at 97.5 81) (size 0.6) (drill 0.3) (layers "F.Cu" "B.Cu") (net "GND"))
 (via (at 87.5 82.75) (size 0.6) (drill 0.3) (layers "F.Cu" "B.Cu") (free yes) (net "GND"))
 (via (at 90.25 93.25) (size 0.6) (drill 0.3) (layers "F.Cu" "B.Cu") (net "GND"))
 (via (at 96 81.75) (size 0.6) (drill 0.3) (layers "F.Cu" "B.Cu") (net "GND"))
 (via (at 90.25 92.5) (size 0.6) (drill 0.3) (layers "F.Cu" "B.Cu") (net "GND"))
 (via (at 88.5 83.5) (size 0.6) (drill 0.3) (layers "F.Cu" "B.Cu") (free yes) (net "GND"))
 (via (at 86 90.25) (size 0.6) (drill 0.3) (layers "F.Cu" "B.Cu") (free yes) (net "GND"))
 (via (at 96.75 81) (size 0.6) (drill 0.3) (layers "F.Cu" "B.Cu") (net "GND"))
 (via (at 86 91) (size 0.6) (drill 0.3) (layers "F.Cu" "B.Cu") (free yes) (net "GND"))
 (via (at 91.5 92.5) (size 0.6) (drill 0.3) (layers "F.Cu" "B.Cu") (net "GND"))
 (via (at 96.75 81.75) (size 0.6) (drill 0.3) (layers "F.Cu" "B.Cu") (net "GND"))
 (via (at 90.25 94) (size 0.6) (drill 0.3) (layers "F.Cu" "B.Cu") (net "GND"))
 (via (at 82.25 85) (size 0.6) (drill 0.3) (layers "F.Cu" "B.Cu") (free yes) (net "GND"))
 (via (at 91.5 93.25) (size 0.6) (drill 0.3) (layers "F.Cu" "B.Cu") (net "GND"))
 (via (at 97.5 82.5) (size 0.6) (drill 0.3) (layers "F.Cu" "B.Cu") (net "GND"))
 (via (at 97.5 81.75) (size 0.6) (drill 0.3) (layers "F.Cu" "B.Cu") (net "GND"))
 (via (at 89 92.5) (size 0.6) (drill 0.3) (layers "F.Cu" "B.Cu") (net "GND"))
 (via (at 88.5 82.75) (size 0.6) (drill 0.3) (layers "F.Cu" "B.Cu") (free yes) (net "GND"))
 (via (at 89 94) (size 0.6) (drill 0.3) (layers "F.Cu" "B.Cu") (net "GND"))
 (via (at 87.5 83.5) (size 0.6) (drill 0.3) (layers "F.Cu" "B.Cu") (free yes) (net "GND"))
 (via (at 83.25 86) (size 0.6) (drill 0.3) (layers "F.Cu" "B.Cu") (free yes) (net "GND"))
 (via (at 96 82.5) (size 0.6) (drill 0.3) (layers "F.Cu" "B.Cu") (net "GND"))
 (via (at 96.75 82.5) (size 0.6) (drill 0.3) (layers "F.Cu" "B.Cu") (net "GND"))
 (via (at 91.5 94) (size 0.6) (drill 0.3) (layers "F.Cu" "B.Cu") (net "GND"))
 (segment (start 93.006823 81.506823) (end 94.522 83.022) (width 0.6) (layer "F.Cu") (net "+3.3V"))
 (segment (start 94.522 83.022) (end 94.522 86.698354) (width 0.6) (layer "F.Cu") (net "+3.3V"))
 (segment (start 88.1625 81.506823) (end 93.006823 81.506823) (width 0.6) (layer "F.Cu") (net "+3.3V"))
 (segment (start 86.195677 87.4125) (end 86.303177 87.305) (width 0.6) (layer "F.Cu") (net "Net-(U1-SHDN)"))
 (segment (start 84.496823 87.4125) (end 86.195677 87.4125) (width 0.6) (layer "F.Cu") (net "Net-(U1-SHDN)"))
 (segment (start 85.493177 81.506823) (end 86.3375 81.506823) (width 0.6) (layer "F.Cu") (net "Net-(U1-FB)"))
 (segment (start 86.3375 81.506823) (end 86.3375 84.960677) (width 0.6) (layer "F.Cu") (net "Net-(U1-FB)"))
 (segment (start 84.575 83.570677) (end 84.575 82.425) (width 0.6) (layer "F.Cu") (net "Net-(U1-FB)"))
 (segment (start 84.575 82.425) (end 85.493177 81.506823) (width 0.6) (layer "F.Cu") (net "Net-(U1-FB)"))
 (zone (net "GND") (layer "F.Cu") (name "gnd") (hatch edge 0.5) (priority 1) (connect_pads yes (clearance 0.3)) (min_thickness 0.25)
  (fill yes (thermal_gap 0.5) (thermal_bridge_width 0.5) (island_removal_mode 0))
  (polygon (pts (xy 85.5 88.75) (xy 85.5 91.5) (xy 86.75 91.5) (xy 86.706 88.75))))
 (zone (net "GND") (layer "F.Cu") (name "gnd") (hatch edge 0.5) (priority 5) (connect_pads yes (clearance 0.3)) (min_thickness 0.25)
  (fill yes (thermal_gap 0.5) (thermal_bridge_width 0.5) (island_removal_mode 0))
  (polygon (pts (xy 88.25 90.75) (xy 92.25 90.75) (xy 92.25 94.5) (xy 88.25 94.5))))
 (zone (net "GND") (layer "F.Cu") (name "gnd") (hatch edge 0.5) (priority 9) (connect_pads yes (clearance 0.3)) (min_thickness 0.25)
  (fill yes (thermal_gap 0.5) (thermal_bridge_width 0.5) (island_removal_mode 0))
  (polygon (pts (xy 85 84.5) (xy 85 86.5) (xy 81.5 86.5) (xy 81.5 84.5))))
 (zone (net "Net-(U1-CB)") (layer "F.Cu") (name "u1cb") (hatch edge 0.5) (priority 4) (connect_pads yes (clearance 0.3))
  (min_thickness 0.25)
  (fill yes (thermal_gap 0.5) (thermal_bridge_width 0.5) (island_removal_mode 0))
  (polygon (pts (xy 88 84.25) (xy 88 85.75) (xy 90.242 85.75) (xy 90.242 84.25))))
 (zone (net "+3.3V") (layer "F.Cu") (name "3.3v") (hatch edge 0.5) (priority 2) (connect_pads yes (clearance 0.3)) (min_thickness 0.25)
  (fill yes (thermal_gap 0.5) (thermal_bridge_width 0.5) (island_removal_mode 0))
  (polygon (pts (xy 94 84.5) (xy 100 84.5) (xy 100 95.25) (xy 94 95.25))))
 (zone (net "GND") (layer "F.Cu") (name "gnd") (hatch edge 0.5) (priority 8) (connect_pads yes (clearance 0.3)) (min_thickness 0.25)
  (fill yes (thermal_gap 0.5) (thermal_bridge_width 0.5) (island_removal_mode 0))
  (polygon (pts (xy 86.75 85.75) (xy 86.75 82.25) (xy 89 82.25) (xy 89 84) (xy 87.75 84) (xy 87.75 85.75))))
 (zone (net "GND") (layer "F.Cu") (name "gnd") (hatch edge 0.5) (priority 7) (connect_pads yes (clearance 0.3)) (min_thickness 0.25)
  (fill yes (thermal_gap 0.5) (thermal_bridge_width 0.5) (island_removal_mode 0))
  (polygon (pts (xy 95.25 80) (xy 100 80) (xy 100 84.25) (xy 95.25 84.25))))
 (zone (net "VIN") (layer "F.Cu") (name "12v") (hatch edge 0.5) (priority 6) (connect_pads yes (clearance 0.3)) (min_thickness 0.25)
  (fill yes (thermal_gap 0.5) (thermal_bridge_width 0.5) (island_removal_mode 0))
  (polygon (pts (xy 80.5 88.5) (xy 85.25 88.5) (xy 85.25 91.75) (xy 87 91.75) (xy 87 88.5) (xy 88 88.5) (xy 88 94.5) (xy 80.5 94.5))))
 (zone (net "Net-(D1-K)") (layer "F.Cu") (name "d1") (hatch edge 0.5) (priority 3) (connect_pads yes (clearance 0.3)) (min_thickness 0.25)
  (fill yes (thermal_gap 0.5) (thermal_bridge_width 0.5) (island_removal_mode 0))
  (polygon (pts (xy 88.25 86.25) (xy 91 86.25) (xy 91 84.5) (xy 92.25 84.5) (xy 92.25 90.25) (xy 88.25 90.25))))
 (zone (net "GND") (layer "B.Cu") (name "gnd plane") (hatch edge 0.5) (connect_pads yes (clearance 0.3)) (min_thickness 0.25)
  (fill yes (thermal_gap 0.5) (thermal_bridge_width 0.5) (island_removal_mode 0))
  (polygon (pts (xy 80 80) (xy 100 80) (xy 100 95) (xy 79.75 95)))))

